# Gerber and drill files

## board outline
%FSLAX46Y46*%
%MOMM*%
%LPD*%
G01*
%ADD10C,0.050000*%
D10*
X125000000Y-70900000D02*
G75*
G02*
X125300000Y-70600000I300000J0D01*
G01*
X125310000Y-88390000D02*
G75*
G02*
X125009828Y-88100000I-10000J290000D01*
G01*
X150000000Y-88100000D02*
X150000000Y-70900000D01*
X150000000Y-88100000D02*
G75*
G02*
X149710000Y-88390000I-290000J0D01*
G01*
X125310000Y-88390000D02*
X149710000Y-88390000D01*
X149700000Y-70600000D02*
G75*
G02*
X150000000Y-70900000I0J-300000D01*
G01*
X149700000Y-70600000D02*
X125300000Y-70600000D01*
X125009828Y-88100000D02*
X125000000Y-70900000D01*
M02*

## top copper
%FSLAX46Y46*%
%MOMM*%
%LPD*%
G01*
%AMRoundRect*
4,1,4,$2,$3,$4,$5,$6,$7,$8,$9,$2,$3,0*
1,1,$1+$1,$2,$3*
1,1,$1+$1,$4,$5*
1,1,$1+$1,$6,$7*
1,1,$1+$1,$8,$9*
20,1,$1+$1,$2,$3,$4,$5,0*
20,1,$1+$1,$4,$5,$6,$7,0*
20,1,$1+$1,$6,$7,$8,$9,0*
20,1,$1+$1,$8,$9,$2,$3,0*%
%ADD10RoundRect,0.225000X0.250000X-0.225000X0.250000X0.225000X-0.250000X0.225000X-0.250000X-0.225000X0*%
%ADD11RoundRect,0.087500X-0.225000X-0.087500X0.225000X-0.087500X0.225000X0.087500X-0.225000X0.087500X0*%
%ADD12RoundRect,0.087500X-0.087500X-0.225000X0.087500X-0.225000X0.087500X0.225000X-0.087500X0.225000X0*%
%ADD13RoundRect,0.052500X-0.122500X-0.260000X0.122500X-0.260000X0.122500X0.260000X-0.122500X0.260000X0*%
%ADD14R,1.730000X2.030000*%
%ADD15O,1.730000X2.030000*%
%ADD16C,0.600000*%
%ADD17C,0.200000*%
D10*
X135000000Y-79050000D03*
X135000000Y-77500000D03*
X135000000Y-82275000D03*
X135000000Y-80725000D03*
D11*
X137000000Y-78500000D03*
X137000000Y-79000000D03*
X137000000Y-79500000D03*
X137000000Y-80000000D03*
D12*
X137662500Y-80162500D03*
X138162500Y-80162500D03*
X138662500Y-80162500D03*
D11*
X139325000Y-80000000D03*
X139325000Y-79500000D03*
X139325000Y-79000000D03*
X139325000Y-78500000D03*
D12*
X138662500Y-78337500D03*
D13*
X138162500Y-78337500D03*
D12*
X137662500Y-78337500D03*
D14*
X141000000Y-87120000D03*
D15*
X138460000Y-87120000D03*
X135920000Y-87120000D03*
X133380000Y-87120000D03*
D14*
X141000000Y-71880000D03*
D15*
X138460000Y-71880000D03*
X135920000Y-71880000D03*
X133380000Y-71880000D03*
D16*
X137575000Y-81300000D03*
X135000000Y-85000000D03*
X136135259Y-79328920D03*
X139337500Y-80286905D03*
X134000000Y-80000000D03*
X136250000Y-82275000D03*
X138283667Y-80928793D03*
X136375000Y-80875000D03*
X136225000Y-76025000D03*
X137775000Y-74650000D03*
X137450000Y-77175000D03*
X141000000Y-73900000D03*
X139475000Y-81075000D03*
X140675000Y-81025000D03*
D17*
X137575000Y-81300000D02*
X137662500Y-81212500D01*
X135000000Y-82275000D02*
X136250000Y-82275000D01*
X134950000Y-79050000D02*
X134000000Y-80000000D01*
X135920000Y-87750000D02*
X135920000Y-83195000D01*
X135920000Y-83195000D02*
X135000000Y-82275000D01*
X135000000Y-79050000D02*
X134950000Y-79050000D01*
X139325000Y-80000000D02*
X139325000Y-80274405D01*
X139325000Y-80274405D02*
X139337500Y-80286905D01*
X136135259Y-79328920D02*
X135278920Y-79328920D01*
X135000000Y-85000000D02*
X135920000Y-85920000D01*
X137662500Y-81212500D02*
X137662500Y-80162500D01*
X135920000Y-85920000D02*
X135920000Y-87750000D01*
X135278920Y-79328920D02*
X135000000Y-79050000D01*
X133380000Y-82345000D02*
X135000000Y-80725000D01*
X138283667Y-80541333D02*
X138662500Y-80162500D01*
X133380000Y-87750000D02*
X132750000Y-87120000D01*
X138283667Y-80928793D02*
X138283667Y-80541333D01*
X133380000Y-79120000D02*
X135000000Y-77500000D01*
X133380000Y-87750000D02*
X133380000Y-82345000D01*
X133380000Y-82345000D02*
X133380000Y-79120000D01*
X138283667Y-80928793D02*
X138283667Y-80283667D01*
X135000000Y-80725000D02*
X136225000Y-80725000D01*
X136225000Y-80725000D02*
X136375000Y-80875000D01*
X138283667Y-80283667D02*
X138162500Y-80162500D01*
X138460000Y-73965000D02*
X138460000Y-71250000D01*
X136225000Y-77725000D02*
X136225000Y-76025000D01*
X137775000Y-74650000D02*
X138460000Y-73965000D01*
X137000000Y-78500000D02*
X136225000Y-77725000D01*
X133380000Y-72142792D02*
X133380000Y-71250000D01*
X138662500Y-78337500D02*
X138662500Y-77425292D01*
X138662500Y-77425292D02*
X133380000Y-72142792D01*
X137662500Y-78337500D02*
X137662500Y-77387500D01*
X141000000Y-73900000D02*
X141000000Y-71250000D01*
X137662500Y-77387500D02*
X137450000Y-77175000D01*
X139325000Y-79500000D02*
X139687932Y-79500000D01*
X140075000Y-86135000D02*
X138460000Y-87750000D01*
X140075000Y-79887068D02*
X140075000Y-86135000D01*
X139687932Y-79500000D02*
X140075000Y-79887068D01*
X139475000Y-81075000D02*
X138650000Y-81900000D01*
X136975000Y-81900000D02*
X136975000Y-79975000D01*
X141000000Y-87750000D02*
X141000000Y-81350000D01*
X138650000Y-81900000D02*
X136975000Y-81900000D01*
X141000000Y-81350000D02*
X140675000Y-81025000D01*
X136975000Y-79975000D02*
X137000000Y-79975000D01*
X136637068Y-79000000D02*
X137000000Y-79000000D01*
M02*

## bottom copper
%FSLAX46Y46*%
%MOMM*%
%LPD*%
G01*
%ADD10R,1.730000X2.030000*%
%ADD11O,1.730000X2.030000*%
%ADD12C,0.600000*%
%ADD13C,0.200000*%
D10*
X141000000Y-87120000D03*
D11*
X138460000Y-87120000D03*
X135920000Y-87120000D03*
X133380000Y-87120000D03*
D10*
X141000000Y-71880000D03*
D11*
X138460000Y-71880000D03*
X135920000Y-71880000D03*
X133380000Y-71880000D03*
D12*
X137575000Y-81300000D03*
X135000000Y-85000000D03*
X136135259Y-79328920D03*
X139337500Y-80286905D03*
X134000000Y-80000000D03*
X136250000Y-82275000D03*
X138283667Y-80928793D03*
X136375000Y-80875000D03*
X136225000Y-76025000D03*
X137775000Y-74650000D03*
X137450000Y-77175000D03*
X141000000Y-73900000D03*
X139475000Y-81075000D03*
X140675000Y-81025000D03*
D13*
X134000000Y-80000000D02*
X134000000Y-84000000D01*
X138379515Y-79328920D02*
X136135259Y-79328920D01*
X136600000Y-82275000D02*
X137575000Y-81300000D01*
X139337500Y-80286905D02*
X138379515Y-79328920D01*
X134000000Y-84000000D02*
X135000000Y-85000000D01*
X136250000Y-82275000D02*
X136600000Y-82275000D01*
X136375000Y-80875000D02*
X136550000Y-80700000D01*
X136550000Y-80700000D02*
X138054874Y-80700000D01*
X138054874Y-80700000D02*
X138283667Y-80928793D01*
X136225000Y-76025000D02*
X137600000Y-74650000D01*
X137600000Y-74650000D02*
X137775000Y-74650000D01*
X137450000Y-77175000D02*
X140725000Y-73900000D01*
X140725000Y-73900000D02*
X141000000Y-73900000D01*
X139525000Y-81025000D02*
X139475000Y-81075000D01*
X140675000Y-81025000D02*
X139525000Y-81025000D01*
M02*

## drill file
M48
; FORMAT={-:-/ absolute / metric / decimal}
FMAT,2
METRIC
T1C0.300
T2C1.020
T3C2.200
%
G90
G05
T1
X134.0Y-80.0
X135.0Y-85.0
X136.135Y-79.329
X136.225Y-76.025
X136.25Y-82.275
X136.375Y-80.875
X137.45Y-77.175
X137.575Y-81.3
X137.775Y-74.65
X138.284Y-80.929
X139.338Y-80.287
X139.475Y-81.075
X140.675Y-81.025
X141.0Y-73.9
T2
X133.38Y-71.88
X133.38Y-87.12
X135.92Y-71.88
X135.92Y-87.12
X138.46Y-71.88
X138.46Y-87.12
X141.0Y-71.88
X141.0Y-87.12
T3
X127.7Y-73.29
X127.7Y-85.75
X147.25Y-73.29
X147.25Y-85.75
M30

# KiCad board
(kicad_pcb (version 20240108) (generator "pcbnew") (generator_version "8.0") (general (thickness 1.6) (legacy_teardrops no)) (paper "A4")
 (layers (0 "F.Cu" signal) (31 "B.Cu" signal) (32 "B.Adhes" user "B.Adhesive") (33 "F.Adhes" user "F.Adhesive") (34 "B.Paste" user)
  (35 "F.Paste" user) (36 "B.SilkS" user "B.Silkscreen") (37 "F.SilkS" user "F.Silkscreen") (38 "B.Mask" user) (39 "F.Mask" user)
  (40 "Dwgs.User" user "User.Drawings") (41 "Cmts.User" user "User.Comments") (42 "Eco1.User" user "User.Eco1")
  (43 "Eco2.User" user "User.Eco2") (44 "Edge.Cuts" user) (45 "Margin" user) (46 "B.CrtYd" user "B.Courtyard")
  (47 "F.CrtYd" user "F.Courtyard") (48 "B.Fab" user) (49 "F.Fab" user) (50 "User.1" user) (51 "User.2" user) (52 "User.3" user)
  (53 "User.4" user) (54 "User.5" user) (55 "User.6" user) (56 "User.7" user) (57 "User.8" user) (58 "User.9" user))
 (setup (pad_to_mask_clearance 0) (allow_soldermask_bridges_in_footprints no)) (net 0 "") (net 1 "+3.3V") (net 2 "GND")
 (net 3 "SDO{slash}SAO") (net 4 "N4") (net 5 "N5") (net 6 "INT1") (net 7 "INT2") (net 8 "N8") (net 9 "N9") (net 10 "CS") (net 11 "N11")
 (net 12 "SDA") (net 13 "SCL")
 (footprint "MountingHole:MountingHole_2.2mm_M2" (layer "F.Cu") (at 127.7 85.75)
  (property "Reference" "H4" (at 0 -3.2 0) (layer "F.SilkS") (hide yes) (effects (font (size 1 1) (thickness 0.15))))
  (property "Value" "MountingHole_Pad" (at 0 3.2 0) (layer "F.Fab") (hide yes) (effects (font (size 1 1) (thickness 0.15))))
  (pad "" np_thru_hole circle (at 0 0) (size 2.2 2.2) (drill 2.2) (layers "*.Cu" "*.Mask")))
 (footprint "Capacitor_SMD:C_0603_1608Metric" (layer "F.Cu") (at 135 78.275 90)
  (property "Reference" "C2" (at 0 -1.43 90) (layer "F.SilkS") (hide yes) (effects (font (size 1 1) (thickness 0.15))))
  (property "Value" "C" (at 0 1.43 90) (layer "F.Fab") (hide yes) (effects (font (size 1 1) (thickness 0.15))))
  (pad "1" smd roundrect (at -0.775 0 90) (size 0.9 0.95) (layers "F.Cu" "F.Paste" "F.Mask") (roundrect_rratio 0.25) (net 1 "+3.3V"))
  (pad "2" smd roundrect (at 0.775 0 90) (size 0.9 0.95) (layers "F.Cu" "F.Paste" "F.Mask") (roundrect_rratio 0.25) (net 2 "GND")))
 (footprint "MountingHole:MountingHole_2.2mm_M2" (layer "F.Cu") (at 147.25 85.75)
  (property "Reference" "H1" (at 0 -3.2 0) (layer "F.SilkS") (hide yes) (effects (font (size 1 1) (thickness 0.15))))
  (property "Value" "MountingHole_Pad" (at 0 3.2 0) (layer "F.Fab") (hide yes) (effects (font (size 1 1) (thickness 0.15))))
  (pad "" np_thru_hole circle (at 0 0) (size 2.2 2.2) (drill 2.2) (layers "*.Cu" "*.Mask")))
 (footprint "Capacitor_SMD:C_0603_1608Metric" (layer "F.Cu") (at 135 81.5 90)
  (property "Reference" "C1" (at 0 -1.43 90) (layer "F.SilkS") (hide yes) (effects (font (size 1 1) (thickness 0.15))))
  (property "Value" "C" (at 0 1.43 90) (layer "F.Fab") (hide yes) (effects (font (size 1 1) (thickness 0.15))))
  (pad "1" smd roundrect (at -0.775 0 90) (size 0.9 0.95) (layers "F.Cu" "F.Paste" "F.Mask") (roundrect_rratio 0.25) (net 1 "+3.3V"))
  (pad "2" smd roundrect (at 0.775 0 90) (size 0.9 0.95) (layers "F.Cu" "F.Paste" "F.Mask") (roundrect_rratio 0.25) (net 2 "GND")))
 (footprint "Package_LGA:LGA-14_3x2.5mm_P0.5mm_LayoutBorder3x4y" (layer "F.Cu") (at 138.1625 79.25)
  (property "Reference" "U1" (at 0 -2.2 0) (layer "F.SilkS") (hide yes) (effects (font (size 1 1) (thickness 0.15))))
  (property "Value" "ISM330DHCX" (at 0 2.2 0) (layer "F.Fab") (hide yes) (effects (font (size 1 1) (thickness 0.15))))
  (pad "1" smd roundrect (at -1.1625 -0.75) (size 0.625 0.35) (layers "F.Cu" "F.Paste" "F.Mask") (roundrect_rratio 0.25)
   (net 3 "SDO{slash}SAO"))
  (pad "2" smd roundrect (at -1.1625 -0.25) (size 0.625 0.35) (layers "F.Cu" "F.Paste" "F.Mask") (roundrect_rratio 0.25) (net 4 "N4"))
  (pad "3" smd roundrect (at -1.1625 0.25) (size 0.625 0.35) (layers "F.Cu" "F.Paste" "F.Mask") (roundrect_rratio 0.25) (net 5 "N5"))
  (pad "4" smd roundrect (at -1.1625 0.75) (size 0.625 0.35) (layers "F.Cu" "F.Paste" "F.Mask") (roundrect_rratio 0.25) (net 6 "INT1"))
  (pad "5" smd roundrect (at -0.5 0.9125) (size 0.35 0.625) (layers "F.Cu" "F.Paste" "F.Mask") (roundrect_rratio 0.25) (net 1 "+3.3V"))
  (pad "6" smd roundrect (at 0 0.9125) (size 0.35 0.625) (layers "F.Cu" "F.Paste" "F.Mask") (roundrect_rratio 0.25) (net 2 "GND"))
  (pad "7" smd roundrect (at 0.5 0.9125) (size 0.35 0.625) (layers "F.Cu" "F.Paste" "F.Mask") (roundrect_rratio 0.25) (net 2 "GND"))
  (pad "8" smd roundrect (at 1.1625 0.75) (size 0.625 0.35) (layers "F.Cu" "F.Paste" "F.Mask") (roundrect_rratio 0.25) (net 1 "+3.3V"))
  (pad "9" smd roundrect (at 1.1625 0.25) (size 0.625 0.35) (layers "F.Cu" "F.Paste" "F.Mask") (roundrect_rratio 0.25) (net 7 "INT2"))
  (pad "10" smd roundrect (at 1.1625 -0.25) (size 0.625 0.35) (layers "F.Cu" "F.Paste" "F.Mask") (roundrect_rratio 0.25) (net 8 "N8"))
  (pad "11" smd roundrect (at 1.1625 -0.75) (size 0.625 0.35) (layers "F.Cu" "F.Paste" "F.Mask") (roundrect_rratio 0.25) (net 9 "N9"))
  (pad "12" smd roundrect (at 0.5 -0.9125) (size 0.35 0.625) (layers "F.Cu" "F.Paste" "F.Mask") (roundrect_rratio 0.25) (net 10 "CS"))
  (pad "13" smd roundrect (at 0 -0.9125) (size 0.35 0.625) (layers "F.Cu" "F.Paste" "F.Mask") (roundrect_rratio 0.15) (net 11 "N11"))
  (pad "14" smd roundrect (at -0.5 -0.9125) (size 0.35 0.625) (layers "F.Cu" "F.Paste" "F.Mask") (roundrect_rratio 0.25) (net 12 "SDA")))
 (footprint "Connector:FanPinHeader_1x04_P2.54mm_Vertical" (layer "F.Cu") (at 141 87.12 180)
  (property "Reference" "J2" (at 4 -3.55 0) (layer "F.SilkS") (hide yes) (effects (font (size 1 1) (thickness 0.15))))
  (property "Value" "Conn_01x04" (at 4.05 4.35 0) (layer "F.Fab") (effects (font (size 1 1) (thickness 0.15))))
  (pad "1" thru_hole rect (at 0 0 270) (size 2.03 1.73) (drill 1.02) (layers "*.Cu" "*.Mask") (remove_unused_layers no) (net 6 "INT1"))
  (pad "2" thru_hole oval (at 2.54 0 270) (size 2.03 1.73) (drill 1.02) (layers "*.Cu" "*.Mask") (remove_unused_layers no) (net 7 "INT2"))
  (pad "3" thru_hole oval (at 5.08 0 270) (size 2.03 1.73) (drill 1.02) (layers "*.Cu" "*.Mask") (remove_unused_layers no) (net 1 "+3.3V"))
  (pad "4" thru_hole oval (at 7.62 0 270) (size 2.03 1.73) (drill 1.02) (layers "*.Cu" "*.Mask") (remove_unused_layers no) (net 2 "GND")))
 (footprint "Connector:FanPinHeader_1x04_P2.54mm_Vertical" (layer "F.Cu") (at 141 71.88 180)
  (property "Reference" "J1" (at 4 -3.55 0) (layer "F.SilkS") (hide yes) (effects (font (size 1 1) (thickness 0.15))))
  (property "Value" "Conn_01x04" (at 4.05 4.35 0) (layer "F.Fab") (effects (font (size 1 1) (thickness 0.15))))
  (pad "1" thru_hole rect (at 0 0 270) (size 2.03 1.73) (drill 1.02) (layers "*.Cu" "*.Mask") (remove_unused_layers no) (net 12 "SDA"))
  (pad "2" thru_hole oval (at 2.54 0 270) (size 2.03 1.73) (drill 1.02) (layers "*.Cu" "*.Mask") (remove_unused_layers no)
   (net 3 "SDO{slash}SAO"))
  (pad "3" thru_hole oval (at 5.08 0 270) (size 2.03 1.73) (drill 1.02) (layers "*.Cu" "*.Mask") (remove_unused_layers no) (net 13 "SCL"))
  (pad "4" thru_hole oval (at 7.62 0 270) (size 2.03 1.73) (drill 1.02) (layers "*.Cu" "*.Mask") (remove_unused_layers no) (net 10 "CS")))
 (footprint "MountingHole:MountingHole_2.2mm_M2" (layer "F.Cu") (at 147.25 73.29)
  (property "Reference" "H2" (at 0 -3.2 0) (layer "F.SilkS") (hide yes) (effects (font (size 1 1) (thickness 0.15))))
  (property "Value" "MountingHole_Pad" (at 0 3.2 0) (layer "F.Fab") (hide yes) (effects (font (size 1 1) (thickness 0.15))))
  (pad "" np_thru_hole circle (at 0 0) (size 2.2 2.2) (drill 2.2) (layers "*.Cu" "*.Mask")))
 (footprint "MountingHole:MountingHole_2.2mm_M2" (layer "F.Cu") (at 127.7 73.29)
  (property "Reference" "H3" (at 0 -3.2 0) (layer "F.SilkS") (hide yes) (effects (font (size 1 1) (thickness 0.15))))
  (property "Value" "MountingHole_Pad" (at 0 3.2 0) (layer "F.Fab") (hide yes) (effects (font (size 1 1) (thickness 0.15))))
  (pad "" np_thru_hole circle (at 0 0) (size 2.2 2.2) (drill 2.2) (layers "*.Cu" "*.Mask")))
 (gr_arc (start 125 70.9) (mid 125.087868 70.687868) (end 125.3 70.6) (stroke (width 0.05) (type default)) (layer "Edge.Cuts"))
 (gr_arc (start 125.31 88.39) (mid 125.098384 88.308688) (end 125.009828 88.1) (stroke (width 0.05) (type default)) (layer "Edge.Cuts"))
 (gr_line (start 150 88.1) (end 150 70.9) (stroke (width 0.05) (type default)) (layer "Edge.Cuts"))
 (gr_arc (start 150 88.1) (mid 149.915061 88.305061) (end 149.71 88.39) (stroke (width 0.05) (type default)) (layer "Edge.Cuts"))
 (gr_line (start 125.31 88.39) (end 149.71 88.39) (stroke (width 0.05) (type default)) (layer "Edge.Cuts"))
 (gr_arc (start 149.7 70.6) (mid 149.912132 70.687868) (end 150 70.9) (stroke (width 0.05) (type default)) (layer "Edge.Cuts"))
 (gr_line (start 149.7 70.6) (end 125.3 70.6) (stroke (width 0.05) (type default)) (layer "Edge.Cuts"))
 (gr_line (start 125.009828 88.1) (end 125 70.9) (stroke (width 0.05) (type default)) (layer "Edge.Cuts"))
 (segment (start 137.575 81.3) (end 137.6625 81.2125) (width 0.2) (layer "F.Cu") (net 1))
 (segment (start 135 82.275) (end 136.25 82.275) (width 0.2) (layer "F.Cu") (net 1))
 (segment (start 134.95 79.05) (end 134 80) (width 0.2) (layer "F.Cu") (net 1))
 (segment (start 135.92 87.75) (end 135.92 83.195) (width 0.2) (layer "F.Cu") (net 1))
 (segment (start 135.92 83.195) (end 135 82.275) (width 0.2) (layer "F.Cu") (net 1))
 (segment (start 135 79.05) (end 134.95 79.05) (width 0.2) (layer "F.Cu") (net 1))
 (segment (start 139.325 80) (end 139.325 80.274405) (width 0.2) (layer "F.Cu") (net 1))
 (segment (start 139.325 80.274405) (end 139.3375 80.286905) (width 0.2) (layer "F.Cu") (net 1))
 (segment (start 136.135259 79.32892) (end 135.27892 79.32892) (width 0.2) (layer "F.Cu") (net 1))
 (segment (start 135 85) (end 135.92 85.92) (width 0.2) (layer "F.Cu") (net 1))
 (segment (start 137.6625 81.2125) (end 137.6625 80.1625) (width 0.2) (layer "F.Cu") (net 1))
 (segment (start 135.92 85.92) (end 135.92 87.75) (width 0.2) (layer "F.Cu") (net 1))
 (segment (start 135.27892 79.32892) (end 135 79.05) (width 0.2) (layer "F.Cu") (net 1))
 (via (at 137.575 81.3) (size 0.6) (drill 0.3) (layers "F.Cu" "B.Cu") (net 1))
 (via (at 135 85) (size 0.6) (drill 0.3) (layers "F.Cu" "B.Cu") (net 1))
 (via (at 136.135259 79.32892) (size 0.6) (drill 0.3) (layers "F.Cu" "B.Cu") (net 1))
 (via (at 139.3375 80.286905) (size 0.6) (drill 0.3) (layers "F.Cu" "B.Cu") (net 1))
 (via (at 134 80) (size 0.6) (drill 0.3) (layers "F.Cu" "B.Cu") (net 1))
 (via (at 136.25 82.275) (size 0.6) (drill 0.3) (layers "F.Cu" "B.Cu") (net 1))
 (segment (start 134 80) (end 134 84) (width 0.2) (layer "B.Cu") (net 1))
 (segment (start 138.379515 79.32892) (end 136.135259 79.32892) (width 0.2) (layer "B.Cu") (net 1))
 (segment (start 136.6 82.275) (end 137.575 81.3) (width 0.2) (layer "B.Cu") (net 1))
 (segment (start 139.3375 80.286905) (end 138.379515 79.32892) (width 0.2) (layer "B.Cu") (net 1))
 (segment (start 134 84) (end 135 85) (width 0.2) (layer "B.Cu") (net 1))
 (segment (start 136.25 82.275) (end 136.6 82.275) (width 0.2) (layer "B.Cu") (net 1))
 (segment (start 133.38 82.345) (end 135 80.725) (width 0.2) (layer "F.Cu") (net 2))
 (segment (start 138.283667 80.541333) (end 138.6625 80.1625) (width 0.2) (layer "F.Cu") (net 2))
 (segment (start 133.38 87.75) (end 132.75 87.12) (width 0.2) (layer "F.Cu") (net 2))
 (segment (start 138.283667 80.928793) (end 138.283667 80.541333) (width 0.2) (layer "F.Cu") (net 2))
 (segment (start 133.38 79.12) (end 135 77.5) (width 0.2) (layer "F.Cu") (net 2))
 (segment (start 133.38 87.75) (end 133.38 82.345) (width 0.2) (layer "F.Cu") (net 2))
 (segment (start 133.38 82.345) (end 133.38 79.12) (width 0.2) (layer "F.Cu") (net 2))
 (segment (start 138.283667 80.928793) (end 138.283667 80.283667) (width 0.2) (layer "F.Cu") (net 2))
 (segment (start 135 80.725) (end 136.225 80.725) (width 0.2) (layer "F.Cu") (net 2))
 (segment (start 136.225 80.725) (end 136.375 80.875) (width 0.2) (layer "F.Cu") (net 2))
 (segment (start 138.283667 80.283667) (end 138.1625 80.1625) (width 0.2) (layer "F.Cu") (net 2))
 (via (at 138.283667 80.928793) (size 0.6) (drill 0.3) (layers "F.Cu" "B.Cu") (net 2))
 (via (at 136.375 80.875) (size 0.6) (drill 0.3) (layers "F.Cu" "B.Cu") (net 2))
 (segment (start 136.375 80.875) (end 136.55 80.7) (width 0.2) (layer "B.Cu") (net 2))
 (segment (start 136.55 80.7) (end 138.054874 80.7) (width 0.2) (layer "B.Cu") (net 2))
 (segment (start 138.054874 80.7) (end 138.283667 80.928793) (width 0.2) (layer "B.Cu") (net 2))
 (segment (start 138.46 73.965) (end 138.46 71.25) (width 0.2) (layer "F.Cu") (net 3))
 (segment (start 136.225 77.725) (end 136.225 76.025) (width 0.2) (layer "F.Cu") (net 3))
 (segment (start 137.775 74.65) (end 138.46 73.965) (width 0.2) (layer "F.Cu") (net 3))
 (segment (start 137 78.5) (end 136.225 77.725) (width 0.2) (layer "F.Cu") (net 3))
 (via (at 136.225 76.025) (size 0.6) (drill 0.3) (layers "F.Cu" "B.Cu") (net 3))
 (via (at 137.775 74.65) (size 0.6) (drill 0.3) (layers "F.Cu" "B.Cu") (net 3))
 (segment (start 136.225 76.025) (end 137.6 74.65) (width 0.2) (layer "B.Cu") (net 3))
 (segment (start 137.6 74.65) (end 137.775 74.65) (width 0.2) (layer "B.Cu") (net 3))
 (segment (start 133.38 72.142792) (end 133.38 71.25) (width 0.2) (layer "F.Cu") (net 10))
 (segment (start 138.6625 78.3375) (end 138.6625 77.425292) (width 0.2) (layer "F.Cu") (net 10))
 (segment (start 138.6625 77.425292) (end 133.38 72.142792) (width 0.2) (layer "F.Cu") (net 10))
 (segment (start 137.6625 78.3375) (end 137.6625 77.3875) (width 0.2) (layer "F.Cu") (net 12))
 (segment (start 141 73.9) (end 141 71.25) (width 0.2) (layer "F.Cu") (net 12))
 (segment (start 137.6625 77.3875) (end 137.45 77.175) (width 0.2) (layer "F.Cu") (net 12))
 (via (at 137.45 77.175) (size 0.6) (drill 0.3) (layers "F.Cu" "B.Cu") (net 12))
 (via (at 141 73.9) (size 0.6) (drill 0.3) (layers "F.Cu" "B.Cu") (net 12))
 (segment (start 137.45 77.175) (end 140.725 73.9) (width 0.2) (layer "B.Cu") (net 12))
 (segment (start 140.725 73.9) (end 141 73.9) (width 0.2) (layer "B.Cu") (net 12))
 (segment (start 139.325 79.5) (end 139.687932 79.5) (width 0.2) (layer "F.Cu") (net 7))
 (segment (start 140.075 86.135) (end 138.46 87.75) (width 0.2) (layer "F.Cu") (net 7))
 (segment (start 140.075 79.887068) (end 140.075 86.135) (width 0.2) (layer "F.Cu") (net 7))
 (segment (start 139.687932 79.5) (end 140.075 79.887068) (width 0.2) (layer "F.Cu") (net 7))
 (segment (start 139.475 81.075) (end 138.65 81.9) (width 0.2) (layer "F.Cu") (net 6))
 (segment (start 136.975 81.9) (end 136.975 79.975) (width 0.2) (layer "F.Cu") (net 6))
 (segment (start 141 87.75) (end 141 81.35) (width 0.2) (layer "F.Cu") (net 6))
 (segment (start 138.65 81.9) (end 136.975 81.9) (width 0.2) (layer "F.Cu") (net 6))
 (segment (start 141 81.35) (end 140.675 81.025) (width 0.2) (layer "F.Cu") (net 6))
 (segment (start 136.975 79.975) (end 137 79.975) (width 0.2) (layer "F.Cu") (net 6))
 (via (at 139.475 81.075) (size 0.6) (drill 0.3) (layers "F.Cu" "B.Cu") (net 6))
 (via (at 140.675 81.025) (size 0.6) (drill 0.3) (layers "F.Cu" "B.Cu") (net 6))
 (segment (start 139.525 81.025) (end 139.475 81.075) (width 0.2) (layer "B.Cu") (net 6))
 (segment (start 140.675 81.025) (end 139.525 81.025) (width 0.2) (layer "B.Cu") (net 6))
 (segment (start 136.637068 79) (end 137 79) (width 0.2) (layer "F.Cu") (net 4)))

